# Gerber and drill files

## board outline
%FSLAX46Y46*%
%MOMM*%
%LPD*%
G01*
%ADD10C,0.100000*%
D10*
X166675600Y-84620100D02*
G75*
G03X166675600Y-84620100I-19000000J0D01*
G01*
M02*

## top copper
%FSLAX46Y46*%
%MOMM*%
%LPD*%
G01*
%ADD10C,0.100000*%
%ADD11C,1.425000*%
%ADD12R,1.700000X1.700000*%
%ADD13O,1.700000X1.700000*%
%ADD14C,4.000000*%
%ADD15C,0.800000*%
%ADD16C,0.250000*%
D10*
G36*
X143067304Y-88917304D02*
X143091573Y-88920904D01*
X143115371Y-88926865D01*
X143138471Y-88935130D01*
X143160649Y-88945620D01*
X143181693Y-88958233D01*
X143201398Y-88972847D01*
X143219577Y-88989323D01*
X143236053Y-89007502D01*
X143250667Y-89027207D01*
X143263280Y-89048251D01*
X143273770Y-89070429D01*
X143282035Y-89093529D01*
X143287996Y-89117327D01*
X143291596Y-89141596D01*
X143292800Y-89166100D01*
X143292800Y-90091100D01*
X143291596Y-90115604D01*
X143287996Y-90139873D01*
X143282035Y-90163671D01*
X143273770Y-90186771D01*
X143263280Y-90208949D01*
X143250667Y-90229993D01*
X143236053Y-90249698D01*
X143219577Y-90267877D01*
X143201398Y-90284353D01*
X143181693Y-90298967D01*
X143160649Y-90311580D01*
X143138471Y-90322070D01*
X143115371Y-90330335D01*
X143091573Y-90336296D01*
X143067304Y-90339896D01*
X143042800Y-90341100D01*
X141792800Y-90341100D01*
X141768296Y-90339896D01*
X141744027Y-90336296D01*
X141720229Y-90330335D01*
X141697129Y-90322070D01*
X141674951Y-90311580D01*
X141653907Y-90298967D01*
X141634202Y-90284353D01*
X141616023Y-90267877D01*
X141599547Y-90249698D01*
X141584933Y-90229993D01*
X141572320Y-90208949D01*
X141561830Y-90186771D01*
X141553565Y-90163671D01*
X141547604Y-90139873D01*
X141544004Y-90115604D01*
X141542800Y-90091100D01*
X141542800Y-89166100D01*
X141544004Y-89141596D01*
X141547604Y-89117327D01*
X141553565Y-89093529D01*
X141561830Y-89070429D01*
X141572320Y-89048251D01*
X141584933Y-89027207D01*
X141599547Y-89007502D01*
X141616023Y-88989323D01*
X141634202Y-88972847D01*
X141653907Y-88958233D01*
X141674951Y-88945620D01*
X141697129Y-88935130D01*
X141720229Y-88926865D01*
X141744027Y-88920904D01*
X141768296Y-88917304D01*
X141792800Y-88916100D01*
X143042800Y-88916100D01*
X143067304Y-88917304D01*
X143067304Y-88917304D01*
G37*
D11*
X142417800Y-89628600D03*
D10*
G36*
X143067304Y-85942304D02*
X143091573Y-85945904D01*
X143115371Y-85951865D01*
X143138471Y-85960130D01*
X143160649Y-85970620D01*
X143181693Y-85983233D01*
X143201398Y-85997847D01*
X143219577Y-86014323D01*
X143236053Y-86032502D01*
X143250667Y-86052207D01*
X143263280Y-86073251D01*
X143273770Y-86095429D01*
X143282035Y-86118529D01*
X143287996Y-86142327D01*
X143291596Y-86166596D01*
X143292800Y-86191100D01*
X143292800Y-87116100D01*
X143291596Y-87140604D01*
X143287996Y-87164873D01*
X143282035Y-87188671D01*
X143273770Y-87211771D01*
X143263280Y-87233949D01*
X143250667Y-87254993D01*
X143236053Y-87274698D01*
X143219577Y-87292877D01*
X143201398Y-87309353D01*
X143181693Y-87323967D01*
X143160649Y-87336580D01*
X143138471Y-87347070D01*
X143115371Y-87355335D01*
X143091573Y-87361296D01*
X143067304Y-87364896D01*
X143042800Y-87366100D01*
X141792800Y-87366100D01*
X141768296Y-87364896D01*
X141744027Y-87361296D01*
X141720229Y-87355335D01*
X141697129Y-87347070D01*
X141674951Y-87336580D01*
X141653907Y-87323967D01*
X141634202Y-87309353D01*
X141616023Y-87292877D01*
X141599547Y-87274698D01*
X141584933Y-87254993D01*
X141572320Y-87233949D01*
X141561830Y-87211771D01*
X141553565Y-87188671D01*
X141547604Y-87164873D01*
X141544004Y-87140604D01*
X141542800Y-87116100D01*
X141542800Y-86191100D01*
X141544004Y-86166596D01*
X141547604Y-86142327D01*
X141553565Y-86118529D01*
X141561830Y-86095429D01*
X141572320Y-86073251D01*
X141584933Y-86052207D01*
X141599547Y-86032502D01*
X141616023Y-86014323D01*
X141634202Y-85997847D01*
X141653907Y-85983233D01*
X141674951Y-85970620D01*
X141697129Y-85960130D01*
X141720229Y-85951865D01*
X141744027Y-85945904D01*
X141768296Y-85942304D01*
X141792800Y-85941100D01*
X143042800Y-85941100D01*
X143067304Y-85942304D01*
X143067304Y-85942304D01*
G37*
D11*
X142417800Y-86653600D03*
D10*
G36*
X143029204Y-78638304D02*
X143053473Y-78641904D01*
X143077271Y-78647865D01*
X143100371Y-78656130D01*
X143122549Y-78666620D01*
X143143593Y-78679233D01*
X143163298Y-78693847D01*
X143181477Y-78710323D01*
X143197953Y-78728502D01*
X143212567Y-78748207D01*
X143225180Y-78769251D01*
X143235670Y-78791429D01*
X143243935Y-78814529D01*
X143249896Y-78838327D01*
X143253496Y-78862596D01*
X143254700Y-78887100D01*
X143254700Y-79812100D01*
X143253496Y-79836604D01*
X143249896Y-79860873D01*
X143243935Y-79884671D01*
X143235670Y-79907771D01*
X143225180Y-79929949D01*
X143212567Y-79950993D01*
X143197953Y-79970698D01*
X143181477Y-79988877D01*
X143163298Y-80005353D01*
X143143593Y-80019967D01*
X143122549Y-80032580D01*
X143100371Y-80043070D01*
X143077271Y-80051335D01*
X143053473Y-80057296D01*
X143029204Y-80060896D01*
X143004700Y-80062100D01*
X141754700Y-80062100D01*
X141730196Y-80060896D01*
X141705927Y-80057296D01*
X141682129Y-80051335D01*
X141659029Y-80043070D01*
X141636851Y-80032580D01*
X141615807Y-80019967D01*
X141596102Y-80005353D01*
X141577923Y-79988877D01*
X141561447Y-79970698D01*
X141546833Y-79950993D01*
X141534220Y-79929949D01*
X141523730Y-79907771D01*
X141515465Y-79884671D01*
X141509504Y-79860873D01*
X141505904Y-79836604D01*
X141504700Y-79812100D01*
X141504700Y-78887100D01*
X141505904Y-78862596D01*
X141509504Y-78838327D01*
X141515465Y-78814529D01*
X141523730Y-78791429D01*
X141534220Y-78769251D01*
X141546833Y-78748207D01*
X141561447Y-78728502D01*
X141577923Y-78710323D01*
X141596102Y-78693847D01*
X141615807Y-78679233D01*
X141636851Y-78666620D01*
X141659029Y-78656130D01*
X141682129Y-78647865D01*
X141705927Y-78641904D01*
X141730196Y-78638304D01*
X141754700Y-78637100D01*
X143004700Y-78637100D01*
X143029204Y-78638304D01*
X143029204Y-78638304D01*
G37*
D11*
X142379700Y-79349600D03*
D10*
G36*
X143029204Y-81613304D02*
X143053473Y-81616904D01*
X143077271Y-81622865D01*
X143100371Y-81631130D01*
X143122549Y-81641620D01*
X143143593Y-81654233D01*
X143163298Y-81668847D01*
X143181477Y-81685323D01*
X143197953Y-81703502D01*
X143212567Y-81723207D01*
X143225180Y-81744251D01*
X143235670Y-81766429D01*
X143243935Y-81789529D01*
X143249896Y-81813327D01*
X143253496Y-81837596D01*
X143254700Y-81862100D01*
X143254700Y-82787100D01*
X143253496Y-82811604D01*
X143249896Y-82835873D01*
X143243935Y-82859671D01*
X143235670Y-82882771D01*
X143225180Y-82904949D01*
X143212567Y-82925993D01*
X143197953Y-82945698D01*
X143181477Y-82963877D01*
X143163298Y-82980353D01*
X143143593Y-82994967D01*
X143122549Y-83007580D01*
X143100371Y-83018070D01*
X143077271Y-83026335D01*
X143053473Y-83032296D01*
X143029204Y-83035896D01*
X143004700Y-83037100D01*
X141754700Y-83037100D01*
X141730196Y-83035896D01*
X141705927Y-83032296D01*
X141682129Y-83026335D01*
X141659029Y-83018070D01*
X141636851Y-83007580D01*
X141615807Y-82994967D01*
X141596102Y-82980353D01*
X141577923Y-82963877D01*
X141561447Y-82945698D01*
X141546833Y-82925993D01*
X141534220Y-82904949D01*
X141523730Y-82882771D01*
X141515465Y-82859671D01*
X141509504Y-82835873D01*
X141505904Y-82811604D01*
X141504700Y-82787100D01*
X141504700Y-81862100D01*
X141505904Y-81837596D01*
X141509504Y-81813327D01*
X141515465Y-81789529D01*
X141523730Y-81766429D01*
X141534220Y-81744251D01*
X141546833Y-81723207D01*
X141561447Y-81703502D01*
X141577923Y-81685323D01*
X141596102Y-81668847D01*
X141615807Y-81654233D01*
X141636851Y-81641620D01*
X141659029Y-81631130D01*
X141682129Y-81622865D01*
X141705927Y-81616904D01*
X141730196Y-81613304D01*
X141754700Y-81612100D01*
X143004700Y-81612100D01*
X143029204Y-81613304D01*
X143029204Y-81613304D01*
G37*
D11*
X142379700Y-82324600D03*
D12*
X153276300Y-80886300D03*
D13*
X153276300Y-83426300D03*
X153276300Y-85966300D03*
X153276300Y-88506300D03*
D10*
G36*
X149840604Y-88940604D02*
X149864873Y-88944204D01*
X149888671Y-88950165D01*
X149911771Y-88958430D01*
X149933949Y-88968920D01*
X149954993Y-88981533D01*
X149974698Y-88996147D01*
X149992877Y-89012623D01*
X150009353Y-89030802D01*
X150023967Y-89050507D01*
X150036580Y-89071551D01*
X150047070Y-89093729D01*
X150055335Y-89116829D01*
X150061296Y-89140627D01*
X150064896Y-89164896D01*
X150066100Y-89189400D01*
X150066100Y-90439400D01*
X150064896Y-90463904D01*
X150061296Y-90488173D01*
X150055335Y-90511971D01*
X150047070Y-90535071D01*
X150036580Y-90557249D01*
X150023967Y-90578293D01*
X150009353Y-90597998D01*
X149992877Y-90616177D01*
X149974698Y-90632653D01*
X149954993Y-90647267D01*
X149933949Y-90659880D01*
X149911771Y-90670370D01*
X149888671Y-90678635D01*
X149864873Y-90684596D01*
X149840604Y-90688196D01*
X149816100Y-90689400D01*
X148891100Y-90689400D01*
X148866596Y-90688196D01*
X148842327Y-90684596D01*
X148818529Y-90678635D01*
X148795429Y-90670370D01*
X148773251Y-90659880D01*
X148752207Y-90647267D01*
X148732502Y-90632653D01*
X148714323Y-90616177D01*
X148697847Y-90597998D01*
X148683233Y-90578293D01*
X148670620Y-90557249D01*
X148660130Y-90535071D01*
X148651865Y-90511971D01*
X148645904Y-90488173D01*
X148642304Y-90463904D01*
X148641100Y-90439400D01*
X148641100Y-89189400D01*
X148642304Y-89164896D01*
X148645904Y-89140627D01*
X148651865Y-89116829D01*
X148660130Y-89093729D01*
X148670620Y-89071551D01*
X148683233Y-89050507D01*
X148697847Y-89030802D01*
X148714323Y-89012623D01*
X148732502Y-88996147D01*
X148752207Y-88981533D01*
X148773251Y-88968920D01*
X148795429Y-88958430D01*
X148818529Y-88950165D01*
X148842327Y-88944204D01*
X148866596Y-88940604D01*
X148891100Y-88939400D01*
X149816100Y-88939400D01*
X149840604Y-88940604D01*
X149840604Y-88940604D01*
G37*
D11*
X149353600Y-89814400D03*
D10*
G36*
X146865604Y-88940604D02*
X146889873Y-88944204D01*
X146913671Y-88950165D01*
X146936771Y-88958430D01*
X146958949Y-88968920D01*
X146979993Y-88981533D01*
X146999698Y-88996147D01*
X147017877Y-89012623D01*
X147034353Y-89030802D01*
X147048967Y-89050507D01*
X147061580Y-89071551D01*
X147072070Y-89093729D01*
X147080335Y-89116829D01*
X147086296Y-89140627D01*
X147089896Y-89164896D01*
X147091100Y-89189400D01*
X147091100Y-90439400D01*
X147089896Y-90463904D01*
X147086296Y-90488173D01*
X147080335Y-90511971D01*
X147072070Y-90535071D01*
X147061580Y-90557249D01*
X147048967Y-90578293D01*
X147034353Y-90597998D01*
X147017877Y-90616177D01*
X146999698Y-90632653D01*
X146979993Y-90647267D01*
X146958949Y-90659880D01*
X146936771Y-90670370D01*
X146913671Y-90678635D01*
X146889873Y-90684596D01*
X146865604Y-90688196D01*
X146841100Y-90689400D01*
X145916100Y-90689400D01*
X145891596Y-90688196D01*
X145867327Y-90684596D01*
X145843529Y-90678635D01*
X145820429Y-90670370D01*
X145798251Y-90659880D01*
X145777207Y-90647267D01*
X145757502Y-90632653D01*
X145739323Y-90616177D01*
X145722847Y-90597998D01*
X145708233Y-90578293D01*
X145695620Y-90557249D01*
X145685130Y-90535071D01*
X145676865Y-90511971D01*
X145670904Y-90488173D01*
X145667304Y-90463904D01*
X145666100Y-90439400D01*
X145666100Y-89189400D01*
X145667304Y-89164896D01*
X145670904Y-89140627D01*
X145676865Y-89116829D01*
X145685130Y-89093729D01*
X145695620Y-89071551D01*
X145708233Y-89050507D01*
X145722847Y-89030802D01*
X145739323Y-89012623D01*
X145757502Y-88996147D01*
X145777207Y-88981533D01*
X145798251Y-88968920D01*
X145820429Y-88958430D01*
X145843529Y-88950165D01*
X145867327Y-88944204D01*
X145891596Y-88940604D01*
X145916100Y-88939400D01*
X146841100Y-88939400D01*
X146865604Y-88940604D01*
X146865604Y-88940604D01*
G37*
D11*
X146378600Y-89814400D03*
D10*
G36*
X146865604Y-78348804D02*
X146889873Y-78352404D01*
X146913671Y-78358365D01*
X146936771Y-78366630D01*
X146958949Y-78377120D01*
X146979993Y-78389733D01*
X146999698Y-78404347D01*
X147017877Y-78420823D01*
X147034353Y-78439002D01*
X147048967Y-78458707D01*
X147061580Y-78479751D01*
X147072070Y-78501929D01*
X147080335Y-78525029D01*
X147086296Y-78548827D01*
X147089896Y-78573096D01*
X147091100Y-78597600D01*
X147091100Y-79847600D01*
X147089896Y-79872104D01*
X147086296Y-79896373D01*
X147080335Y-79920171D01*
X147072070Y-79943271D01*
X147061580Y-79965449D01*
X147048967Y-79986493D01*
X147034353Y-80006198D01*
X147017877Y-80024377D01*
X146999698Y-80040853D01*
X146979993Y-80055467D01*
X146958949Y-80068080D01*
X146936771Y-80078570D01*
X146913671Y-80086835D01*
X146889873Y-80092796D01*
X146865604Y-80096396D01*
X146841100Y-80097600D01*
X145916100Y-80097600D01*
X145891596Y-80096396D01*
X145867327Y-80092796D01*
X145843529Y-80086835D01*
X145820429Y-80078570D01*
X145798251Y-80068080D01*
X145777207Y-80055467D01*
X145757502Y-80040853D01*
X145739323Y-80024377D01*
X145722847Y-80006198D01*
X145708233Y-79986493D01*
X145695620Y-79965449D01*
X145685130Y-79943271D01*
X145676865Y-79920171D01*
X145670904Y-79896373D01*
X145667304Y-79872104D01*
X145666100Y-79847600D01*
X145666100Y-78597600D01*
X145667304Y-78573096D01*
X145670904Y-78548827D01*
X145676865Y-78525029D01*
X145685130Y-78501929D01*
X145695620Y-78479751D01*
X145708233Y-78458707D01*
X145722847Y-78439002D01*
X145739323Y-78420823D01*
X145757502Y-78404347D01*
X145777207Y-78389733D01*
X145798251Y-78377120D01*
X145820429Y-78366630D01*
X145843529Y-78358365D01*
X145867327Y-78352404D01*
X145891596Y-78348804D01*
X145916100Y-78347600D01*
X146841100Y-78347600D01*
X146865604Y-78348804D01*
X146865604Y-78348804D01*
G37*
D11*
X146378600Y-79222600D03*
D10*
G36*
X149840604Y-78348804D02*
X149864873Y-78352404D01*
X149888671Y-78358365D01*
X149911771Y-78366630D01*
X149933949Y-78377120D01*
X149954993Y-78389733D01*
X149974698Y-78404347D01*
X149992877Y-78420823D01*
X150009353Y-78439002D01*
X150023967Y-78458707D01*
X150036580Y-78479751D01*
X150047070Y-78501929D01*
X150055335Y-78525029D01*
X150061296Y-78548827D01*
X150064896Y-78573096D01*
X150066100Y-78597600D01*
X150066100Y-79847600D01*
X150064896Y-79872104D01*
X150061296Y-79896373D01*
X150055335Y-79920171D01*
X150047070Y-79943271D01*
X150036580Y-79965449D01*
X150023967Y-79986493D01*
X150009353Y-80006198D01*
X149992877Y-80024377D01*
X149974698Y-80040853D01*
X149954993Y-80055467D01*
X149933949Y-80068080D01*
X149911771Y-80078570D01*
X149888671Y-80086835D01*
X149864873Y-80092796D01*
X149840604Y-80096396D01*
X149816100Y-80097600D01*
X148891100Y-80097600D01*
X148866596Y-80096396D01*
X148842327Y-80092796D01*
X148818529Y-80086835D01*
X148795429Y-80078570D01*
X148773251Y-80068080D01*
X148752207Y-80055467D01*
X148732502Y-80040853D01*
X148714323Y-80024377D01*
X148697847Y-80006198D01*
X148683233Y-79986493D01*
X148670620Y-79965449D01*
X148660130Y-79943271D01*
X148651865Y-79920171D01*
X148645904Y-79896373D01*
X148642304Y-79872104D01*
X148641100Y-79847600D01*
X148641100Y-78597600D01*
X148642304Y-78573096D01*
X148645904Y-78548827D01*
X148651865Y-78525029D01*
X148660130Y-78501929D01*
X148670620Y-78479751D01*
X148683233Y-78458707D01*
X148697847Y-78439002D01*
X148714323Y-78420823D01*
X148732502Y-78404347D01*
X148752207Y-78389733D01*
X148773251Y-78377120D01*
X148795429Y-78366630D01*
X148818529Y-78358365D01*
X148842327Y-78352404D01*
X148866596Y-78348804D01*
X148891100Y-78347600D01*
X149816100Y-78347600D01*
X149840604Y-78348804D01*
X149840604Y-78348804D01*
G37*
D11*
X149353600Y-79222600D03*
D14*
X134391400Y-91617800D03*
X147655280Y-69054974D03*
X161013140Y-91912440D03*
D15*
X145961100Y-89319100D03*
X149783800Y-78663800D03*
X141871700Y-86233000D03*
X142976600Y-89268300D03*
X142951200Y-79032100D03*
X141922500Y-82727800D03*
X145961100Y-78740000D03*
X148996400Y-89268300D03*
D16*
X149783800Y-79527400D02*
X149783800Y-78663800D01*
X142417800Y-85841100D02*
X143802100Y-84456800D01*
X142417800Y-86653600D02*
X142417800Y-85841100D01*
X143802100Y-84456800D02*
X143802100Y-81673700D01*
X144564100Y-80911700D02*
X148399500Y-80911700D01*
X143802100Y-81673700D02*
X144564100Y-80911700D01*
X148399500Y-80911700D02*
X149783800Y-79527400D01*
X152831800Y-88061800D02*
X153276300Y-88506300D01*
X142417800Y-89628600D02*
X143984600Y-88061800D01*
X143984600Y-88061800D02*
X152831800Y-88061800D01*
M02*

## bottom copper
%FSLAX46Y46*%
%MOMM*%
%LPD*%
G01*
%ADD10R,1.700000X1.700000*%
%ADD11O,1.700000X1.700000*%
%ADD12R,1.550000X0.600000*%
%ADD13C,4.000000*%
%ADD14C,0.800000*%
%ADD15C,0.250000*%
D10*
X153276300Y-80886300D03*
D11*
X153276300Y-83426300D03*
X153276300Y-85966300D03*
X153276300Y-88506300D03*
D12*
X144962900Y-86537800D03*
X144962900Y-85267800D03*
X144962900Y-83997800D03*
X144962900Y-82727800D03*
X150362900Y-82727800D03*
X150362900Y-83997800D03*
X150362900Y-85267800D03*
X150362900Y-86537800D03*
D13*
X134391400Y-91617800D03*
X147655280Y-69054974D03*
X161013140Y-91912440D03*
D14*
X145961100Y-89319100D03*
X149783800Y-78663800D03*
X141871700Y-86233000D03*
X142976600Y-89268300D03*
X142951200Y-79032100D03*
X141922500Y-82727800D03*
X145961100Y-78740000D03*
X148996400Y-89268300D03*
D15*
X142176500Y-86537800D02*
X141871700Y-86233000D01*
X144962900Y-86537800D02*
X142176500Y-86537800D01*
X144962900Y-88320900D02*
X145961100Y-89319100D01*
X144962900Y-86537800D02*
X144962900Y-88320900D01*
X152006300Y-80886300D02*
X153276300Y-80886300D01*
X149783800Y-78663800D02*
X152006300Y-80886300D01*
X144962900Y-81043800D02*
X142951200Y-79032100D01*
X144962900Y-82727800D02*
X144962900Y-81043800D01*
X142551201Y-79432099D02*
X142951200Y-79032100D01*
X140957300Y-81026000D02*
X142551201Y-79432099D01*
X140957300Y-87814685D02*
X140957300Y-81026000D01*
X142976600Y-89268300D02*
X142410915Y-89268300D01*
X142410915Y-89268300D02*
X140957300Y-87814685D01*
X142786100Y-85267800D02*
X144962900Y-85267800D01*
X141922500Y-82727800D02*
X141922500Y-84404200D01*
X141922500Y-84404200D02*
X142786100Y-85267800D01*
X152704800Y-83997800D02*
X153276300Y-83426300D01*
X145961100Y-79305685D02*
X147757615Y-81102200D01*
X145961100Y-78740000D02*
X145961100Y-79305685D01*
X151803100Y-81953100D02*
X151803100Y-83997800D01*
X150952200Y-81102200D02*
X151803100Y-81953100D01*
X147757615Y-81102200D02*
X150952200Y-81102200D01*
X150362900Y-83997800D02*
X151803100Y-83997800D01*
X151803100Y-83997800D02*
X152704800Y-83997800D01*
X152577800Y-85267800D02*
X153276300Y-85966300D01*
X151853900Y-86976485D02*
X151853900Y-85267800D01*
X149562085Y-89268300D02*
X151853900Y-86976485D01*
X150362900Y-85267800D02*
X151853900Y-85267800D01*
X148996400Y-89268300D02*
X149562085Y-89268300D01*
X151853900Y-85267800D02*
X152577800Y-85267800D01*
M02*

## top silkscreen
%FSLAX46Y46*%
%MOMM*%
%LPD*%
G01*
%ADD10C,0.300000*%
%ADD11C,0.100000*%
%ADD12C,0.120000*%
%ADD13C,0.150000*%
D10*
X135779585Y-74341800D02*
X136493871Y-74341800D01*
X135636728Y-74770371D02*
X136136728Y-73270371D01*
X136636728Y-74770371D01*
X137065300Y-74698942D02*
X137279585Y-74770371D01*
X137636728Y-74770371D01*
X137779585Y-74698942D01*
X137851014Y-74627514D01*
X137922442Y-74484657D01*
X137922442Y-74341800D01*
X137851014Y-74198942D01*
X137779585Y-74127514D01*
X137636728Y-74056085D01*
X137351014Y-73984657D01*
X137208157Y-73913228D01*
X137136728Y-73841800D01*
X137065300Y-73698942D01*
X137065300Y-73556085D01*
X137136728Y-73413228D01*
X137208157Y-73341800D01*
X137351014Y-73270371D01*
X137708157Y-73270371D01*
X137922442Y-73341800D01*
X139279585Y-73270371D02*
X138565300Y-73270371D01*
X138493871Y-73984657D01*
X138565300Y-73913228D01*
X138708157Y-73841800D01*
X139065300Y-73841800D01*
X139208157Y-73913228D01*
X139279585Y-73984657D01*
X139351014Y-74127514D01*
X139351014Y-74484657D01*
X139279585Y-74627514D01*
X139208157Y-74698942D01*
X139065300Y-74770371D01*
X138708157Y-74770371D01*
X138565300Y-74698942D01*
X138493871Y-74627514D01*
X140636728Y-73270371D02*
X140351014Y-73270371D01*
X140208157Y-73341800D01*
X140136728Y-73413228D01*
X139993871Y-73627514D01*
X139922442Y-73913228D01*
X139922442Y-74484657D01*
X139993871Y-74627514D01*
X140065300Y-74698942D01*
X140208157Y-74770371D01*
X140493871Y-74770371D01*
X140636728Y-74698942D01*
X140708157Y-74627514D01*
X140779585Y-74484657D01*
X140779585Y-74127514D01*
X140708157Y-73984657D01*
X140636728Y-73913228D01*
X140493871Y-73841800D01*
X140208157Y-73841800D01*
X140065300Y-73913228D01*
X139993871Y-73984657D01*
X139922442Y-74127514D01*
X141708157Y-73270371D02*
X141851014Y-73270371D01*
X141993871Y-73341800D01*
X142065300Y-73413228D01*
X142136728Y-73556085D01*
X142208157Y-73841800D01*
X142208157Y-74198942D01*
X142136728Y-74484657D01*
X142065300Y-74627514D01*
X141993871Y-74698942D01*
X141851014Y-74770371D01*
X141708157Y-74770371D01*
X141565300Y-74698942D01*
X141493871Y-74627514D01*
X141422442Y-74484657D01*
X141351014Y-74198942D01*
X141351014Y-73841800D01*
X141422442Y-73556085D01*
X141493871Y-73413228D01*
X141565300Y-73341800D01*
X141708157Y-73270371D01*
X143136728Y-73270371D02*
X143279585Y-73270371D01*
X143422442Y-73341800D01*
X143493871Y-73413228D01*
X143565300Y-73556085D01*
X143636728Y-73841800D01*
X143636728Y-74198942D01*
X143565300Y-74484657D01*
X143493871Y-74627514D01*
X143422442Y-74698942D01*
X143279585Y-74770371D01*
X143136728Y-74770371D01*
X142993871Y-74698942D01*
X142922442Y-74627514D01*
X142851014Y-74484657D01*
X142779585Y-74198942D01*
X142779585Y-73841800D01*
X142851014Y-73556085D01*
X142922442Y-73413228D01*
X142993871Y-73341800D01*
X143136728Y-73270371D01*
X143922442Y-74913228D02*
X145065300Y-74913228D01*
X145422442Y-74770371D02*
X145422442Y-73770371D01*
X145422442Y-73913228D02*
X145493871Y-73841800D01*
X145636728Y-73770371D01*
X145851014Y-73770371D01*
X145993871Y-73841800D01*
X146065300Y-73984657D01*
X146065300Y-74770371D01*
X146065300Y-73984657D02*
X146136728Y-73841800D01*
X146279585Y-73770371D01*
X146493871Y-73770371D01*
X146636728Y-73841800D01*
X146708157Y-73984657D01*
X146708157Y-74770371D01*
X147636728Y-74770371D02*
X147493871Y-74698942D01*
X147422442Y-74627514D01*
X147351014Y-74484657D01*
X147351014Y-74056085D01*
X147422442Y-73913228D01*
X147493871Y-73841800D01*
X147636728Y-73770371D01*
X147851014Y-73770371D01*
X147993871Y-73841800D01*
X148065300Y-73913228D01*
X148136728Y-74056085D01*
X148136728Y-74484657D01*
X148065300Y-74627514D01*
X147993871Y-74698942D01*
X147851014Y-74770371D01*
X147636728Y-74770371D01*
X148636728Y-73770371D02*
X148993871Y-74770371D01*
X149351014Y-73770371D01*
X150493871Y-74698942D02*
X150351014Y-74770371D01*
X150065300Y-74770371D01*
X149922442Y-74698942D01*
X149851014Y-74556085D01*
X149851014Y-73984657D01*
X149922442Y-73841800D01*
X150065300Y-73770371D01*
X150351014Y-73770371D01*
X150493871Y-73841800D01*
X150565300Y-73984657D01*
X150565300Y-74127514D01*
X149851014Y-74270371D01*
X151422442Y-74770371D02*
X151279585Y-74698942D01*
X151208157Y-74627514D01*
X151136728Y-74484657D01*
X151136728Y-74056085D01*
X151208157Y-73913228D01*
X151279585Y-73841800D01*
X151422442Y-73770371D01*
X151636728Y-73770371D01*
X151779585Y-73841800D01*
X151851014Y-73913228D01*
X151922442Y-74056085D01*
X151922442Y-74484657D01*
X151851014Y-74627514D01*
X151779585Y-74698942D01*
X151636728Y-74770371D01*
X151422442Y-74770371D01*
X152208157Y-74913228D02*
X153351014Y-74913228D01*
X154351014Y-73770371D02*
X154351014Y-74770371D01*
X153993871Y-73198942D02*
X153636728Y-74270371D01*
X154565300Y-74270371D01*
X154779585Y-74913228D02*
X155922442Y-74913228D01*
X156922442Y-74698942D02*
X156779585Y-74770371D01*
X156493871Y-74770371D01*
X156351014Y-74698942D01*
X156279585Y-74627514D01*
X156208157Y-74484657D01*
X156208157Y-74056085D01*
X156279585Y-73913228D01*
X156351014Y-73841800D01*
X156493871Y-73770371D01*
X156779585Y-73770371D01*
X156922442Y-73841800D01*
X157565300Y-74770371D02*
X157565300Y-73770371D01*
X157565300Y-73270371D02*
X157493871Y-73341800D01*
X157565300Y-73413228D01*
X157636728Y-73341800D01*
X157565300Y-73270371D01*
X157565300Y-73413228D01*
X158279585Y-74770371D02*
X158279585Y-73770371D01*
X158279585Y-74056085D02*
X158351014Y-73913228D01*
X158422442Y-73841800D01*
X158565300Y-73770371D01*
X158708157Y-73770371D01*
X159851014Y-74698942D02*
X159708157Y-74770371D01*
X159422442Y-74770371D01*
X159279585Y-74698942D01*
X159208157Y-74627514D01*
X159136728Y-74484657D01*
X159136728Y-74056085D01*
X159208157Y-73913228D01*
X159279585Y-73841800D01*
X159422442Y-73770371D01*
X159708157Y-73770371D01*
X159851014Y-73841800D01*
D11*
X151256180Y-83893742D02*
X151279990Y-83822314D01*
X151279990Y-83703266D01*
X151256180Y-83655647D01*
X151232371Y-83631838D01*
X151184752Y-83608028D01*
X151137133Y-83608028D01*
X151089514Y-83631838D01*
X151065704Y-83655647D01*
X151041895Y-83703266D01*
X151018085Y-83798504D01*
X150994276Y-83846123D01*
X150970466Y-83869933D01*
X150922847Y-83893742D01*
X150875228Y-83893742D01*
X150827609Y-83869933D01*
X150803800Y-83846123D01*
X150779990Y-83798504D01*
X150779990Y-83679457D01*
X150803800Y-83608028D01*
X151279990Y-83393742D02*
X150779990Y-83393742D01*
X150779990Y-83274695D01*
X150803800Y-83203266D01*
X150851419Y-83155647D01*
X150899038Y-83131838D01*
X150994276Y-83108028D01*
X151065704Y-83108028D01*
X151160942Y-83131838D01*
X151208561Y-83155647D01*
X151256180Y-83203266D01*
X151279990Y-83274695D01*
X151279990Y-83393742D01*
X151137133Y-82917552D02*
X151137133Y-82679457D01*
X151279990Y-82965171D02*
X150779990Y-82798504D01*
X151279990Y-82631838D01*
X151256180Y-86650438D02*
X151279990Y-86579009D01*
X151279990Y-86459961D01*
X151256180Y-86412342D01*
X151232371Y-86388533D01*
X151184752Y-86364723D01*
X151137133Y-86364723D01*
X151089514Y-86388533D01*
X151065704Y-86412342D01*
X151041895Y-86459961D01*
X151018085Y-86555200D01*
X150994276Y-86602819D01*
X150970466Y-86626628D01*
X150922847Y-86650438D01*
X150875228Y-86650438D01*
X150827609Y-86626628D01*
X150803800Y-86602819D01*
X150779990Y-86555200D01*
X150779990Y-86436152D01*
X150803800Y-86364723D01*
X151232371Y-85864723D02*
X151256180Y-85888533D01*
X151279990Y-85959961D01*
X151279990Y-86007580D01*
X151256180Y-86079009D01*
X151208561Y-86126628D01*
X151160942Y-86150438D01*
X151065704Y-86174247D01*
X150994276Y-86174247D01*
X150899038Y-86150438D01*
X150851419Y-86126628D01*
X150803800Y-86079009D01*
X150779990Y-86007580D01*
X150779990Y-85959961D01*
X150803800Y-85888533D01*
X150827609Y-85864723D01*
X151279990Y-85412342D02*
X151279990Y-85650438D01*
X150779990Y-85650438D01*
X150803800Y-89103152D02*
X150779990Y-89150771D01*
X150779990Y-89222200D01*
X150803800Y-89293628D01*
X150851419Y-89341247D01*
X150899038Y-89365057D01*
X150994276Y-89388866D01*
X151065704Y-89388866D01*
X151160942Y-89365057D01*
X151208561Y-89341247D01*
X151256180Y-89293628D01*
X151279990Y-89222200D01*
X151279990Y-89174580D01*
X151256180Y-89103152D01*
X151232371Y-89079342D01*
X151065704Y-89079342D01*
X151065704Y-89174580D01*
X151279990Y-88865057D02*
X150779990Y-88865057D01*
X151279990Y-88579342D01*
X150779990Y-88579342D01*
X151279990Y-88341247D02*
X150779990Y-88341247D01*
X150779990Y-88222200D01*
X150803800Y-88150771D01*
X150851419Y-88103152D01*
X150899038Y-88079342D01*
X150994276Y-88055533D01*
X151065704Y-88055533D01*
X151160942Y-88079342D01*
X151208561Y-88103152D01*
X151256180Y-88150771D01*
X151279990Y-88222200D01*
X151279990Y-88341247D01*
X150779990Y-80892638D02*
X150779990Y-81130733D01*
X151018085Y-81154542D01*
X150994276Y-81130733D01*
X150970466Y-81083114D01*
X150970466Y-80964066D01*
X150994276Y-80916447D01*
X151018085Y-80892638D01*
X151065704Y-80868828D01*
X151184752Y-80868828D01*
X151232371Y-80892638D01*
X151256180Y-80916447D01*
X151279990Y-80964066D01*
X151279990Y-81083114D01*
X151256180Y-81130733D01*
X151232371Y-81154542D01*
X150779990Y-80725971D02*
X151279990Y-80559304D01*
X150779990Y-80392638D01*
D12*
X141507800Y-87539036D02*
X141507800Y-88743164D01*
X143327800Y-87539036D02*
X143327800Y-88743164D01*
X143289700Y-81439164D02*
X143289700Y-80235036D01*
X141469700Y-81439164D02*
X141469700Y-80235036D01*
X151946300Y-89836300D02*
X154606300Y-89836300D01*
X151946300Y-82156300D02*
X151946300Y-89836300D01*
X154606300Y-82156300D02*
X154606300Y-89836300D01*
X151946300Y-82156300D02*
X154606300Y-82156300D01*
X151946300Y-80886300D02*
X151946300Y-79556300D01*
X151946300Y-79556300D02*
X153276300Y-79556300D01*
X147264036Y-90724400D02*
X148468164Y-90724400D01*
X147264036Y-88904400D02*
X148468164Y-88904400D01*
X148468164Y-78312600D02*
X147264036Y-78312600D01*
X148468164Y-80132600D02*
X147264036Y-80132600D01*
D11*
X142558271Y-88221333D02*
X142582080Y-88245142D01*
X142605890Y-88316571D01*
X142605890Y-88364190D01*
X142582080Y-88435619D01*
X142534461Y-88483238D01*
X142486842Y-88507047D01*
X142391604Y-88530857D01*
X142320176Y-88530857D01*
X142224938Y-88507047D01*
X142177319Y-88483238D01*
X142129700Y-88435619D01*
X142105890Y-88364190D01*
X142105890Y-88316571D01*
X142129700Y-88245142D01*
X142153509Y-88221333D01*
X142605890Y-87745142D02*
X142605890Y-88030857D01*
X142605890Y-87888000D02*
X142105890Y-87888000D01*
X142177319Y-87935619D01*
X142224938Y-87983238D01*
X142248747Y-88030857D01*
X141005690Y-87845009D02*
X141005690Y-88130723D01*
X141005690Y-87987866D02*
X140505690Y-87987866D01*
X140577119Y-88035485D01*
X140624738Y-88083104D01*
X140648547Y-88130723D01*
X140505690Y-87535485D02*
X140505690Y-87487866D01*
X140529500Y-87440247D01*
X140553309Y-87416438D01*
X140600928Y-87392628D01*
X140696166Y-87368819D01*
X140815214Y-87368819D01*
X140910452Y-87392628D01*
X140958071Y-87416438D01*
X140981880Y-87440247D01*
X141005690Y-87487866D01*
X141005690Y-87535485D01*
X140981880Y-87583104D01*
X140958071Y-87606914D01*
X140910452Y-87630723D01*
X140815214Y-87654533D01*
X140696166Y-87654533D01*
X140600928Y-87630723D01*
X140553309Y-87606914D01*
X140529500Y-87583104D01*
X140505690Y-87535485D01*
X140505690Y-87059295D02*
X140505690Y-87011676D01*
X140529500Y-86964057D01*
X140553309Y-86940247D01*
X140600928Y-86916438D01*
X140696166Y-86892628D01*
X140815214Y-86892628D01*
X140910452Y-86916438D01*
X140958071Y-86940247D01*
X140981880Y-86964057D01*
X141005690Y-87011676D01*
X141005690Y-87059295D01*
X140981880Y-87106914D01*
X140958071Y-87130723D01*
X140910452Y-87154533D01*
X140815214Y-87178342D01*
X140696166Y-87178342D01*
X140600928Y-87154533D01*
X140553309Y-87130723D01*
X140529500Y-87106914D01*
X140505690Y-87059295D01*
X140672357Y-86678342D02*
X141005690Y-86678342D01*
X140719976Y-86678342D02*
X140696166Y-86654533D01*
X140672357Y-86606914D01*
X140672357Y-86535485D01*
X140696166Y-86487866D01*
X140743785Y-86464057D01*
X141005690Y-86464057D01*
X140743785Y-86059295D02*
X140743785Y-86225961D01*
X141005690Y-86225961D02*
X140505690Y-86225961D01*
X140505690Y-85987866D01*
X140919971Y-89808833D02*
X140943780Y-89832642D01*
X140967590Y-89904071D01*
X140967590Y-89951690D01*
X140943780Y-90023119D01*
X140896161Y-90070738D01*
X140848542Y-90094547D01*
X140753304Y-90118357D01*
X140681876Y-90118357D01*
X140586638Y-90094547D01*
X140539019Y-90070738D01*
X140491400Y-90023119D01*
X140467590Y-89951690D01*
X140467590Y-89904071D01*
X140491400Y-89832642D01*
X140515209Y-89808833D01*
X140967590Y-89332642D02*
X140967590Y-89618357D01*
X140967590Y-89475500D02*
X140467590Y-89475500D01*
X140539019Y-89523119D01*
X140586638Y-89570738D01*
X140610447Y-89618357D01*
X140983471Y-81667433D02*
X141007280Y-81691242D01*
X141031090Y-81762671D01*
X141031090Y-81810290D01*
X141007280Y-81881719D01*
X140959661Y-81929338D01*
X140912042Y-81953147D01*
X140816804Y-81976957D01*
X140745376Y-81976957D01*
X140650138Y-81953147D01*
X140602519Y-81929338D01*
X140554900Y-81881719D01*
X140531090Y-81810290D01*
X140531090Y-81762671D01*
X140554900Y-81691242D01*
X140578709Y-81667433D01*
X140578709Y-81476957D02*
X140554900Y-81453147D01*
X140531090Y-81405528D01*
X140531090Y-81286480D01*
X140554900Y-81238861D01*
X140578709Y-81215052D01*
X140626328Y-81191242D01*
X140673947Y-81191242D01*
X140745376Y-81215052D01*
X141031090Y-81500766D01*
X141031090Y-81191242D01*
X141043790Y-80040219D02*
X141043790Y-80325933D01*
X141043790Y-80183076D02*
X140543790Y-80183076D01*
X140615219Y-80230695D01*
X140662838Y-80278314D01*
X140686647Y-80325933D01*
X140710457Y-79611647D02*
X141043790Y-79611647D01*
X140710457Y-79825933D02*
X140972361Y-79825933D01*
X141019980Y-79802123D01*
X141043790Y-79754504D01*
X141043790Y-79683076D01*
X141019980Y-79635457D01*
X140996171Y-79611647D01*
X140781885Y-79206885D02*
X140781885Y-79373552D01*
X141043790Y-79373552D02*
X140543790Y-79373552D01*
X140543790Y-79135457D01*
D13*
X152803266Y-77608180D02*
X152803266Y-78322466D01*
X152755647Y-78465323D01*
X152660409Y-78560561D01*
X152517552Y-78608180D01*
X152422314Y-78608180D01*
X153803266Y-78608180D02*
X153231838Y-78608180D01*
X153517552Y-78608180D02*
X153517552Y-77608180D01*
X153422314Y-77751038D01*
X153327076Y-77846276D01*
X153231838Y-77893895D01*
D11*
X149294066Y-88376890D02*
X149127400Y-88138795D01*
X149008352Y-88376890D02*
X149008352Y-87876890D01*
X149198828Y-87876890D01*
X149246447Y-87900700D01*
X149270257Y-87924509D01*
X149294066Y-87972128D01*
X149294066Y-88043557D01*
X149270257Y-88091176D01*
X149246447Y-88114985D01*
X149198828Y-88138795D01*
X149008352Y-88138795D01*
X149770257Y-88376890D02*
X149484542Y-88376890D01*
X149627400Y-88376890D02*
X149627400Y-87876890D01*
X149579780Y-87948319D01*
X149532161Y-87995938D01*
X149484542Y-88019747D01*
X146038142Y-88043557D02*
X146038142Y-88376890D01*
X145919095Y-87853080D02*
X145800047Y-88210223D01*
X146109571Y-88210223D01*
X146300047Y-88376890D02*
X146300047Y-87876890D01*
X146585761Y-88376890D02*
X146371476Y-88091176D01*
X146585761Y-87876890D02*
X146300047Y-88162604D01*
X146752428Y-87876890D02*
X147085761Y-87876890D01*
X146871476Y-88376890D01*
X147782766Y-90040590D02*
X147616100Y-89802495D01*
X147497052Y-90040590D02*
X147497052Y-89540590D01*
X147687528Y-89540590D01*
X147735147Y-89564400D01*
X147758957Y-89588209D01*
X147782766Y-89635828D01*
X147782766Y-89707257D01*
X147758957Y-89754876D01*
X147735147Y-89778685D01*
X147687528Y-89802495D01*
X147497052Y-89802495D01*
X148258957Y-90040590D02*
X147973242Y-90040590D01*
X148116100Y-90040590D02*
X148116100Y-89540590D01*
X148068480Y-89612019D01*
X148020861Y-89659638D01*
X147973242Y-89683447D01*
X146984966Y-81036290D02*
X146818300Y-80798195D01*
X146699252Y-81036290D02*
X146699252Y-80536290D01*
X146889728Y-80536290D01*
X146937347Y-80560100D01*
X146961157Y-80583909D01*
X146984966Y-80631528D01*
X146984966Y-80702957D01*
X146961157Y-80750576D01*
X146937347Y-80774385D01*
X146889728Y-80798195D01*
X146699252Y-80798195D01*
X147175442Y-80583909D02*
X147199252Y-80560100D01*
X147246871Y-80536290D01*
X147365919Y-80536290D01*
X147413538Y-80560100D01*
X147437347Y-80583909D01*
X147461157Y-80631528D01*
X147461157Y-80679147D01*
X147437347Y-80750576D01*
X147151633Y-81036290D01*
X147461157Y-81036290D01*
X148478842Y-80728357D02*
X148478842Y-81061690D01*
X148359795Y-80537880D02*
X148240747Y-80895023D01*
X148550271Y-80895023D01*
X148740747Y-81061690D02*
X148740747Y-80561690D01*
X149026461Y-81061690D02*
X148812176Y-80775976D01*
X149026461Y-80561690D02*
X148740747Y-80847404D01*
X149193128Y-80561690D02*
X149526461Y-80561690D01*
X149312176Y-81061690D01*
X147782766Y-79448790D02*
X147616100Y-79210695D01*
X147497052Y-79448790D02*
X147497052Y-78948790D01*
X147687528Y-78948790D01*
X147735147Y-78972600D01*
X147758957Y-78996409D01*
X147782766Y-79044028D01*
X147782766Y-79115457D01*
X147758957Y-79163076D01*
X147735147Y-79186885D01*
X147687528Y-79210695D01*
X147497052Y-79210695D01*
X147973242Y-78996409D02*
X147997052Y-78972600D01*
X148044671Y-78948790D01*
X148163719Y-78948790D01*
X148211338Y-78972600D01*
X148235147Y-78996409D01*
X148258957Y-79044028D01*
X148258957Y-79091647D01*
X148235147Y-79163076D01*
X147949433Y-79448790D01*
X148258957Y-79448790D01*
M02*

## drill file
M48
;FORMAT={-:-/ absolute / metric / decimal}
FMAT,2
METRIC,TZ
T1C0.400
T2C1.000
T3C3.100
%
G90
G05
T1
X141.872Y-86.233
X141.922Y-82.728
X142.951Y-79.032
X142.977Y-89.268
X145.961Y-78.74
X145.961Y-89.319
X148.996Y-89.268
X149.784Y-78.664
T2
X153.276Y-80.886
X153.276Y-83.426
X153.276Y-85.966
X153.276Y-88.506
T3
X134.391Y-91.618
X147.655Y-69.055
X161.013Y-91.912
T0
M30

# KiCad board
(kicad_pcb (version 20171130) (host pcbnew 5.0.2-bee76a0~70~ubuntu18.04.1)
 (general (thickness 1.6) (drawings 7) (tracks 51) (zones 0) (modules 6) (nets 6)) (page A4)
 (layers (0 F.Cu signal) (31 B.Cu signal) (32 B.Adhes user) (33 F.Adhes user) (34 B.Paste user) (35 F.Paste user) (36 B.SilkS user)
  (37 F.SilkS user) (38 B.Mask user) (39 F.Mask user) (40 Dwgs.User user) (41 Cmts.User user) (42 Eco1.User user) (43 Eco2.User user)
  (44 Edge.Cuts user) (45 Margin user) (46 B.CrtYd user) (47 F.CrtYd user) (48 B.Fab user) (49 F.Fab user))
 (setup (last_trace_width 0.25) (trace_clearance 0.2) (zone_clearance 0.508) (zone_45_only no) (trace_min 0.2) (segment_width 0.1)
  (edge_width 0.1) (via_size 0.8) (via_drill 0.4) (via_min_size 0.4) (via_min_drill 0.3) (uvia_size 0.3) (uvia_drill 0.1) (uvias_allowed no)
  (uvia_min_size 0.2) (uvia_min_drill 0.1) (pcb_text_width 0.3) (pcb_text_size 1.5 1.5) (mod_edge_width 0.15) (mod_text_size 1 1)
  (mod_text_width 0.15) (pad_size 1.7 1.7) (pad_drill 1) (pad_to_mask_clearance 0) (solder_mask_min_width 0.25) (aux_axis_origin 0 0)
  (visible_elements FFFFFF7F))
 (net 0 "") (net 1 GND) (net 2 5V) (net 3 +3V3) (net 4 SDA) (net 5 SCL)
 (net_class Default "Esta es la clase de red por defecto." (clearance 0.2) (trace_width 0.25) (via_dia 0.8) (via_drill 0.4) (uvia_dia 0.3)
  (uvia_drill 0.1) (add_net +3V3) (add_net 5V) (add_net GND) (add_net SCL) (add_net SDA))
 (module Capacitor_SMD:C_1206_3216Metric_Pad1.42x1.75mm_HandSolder (layer F.Cu) (at 142.4178 88.1411 270)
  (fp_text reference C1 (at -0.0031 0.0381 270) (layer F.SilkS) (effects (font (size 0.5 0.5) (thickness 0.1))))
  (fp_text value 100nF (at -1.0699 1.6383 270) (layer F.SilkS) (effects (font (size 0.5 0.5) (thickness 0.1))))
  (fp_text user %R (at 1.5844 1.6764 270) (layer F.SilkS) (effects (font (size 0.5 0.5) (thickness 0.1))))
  (fp_line (start -0.602064 0.91) (end 0.602064 0.91) (layer F.SilkS) (width 0.12))
  (fp_line (start -0.602064 -0.91) (end 0.602064 -0.91) (layer F.SilkS) (width 0.12))
  (pad 2 smd roundrect (at 1.4875 0 270) (size 1.425 1.75) (layers F.Cu F.Paste F.Mask) (roundrect_rratio 0.175439) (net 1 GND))
  (pad 1 smd roundrect (at -1.4875 0 270) (size 1.425 1.75) (layers F.Cu F.Paste F.Mask) (roundrect_rratio 0.175439) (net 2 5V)))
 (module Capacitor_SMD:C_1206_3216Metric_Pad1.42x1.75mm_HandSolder (layer F.Cu) (at 142.3797 80.8371 90)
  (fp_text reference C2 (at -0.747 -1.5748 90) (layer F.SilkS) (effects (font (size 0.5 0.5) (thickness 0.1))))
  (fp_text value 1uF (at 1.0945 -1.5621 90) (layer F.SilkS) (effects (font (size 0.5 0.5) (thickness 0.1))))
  (fp_line (start -0.602064 0.91) (end 0.602064 0.91) (layer F.SilkS) (width 0.12))
  (fp_line (start -0.602064 -0.91) (end 0.602064 -0.91) (layer F.SilkS) (width 0.12))
  (pad 2 smd roundrect (at 1.4875 0 90) (size 1.425 1.75) (layers F.Cu F.Paste F.Mask) (roundrect_rratio 0.175439) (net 1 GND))
  (pad 1 smd roundrect (at -1.4875 0 90) (size 1.425 1.75) (layers F.Cu F.Paste F.Mask) (roundrect_rratio 0.175439) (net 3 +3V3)))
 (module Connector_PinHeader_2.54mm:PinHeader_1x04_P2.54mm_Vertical (layer F.Cu) (at 153.2763 80.8863)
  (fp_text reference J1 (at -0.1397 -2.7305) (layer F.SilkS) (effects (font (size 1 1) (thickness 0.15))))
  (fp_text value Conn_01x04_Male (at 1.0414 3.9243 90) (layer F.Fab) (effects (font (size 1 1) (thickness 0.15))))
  (fp_line (start -1.33 8.95) (end 1.33 8.95) (layer F.SilkS) (width 0.12))
  (fp_line (start -1.33 1.27) (end -1.33 8.95) (layer F.SilkS) (width 0.12))
  (fp_line (start 1.33 1.27) (end 1.33 8.95) (layer F.SilkS) (width 0.12))
  (fp_line (start -1.33 1.27) (end 1.33 1.27) (layer F.SilkS) (width 0.12))
  (fp_line (start -1.33 0) (end -1.33 -1.33) (layer F.SilkS) (width 0.12))
  (fp_line (start -1.33 -1.33) (end 0 -1.33) (layer F.SilkS) (width 0.12))
  (pad 1 thru_hole rect (at 0 0) (size 1.7 1.7) (drill 1) (layers *.Cu *.Mask) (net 2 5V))
  (pad 2 thru_hole oval (at 0 2.54) (size 1.7 1.7) (drill 1) (layers *.Cu *.Mask) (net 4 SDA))
  (pad 3 thru_hole oval (at 0 5.08) (size 1.7 1.7) (drill 1) (layers *.Cu *.Mask) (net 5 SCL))
  (pad 4 thru_hole oval (at 0 7.62) (size 1.7 1.7) (drill 1) (layers *.Cu *.Mask) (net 1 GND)))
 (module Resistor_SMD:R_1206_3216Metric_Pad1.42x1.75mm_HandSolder (layer F.Cu) (at 147.8661 89.8144)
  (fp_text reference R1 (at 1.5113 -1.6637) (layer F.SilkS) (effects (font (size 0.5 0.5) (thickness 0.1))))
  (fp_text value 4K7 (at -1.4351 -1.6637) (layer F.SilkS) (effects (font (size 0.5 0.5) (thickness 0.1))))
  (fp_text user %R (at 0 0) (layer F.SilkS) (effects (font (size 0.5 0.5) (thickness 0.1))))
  (fp_line (start -0.602064 0.91) (end 0.602064 0.91) (layer F.SilkS) (width 0.12))
  (fp_line (start -0.602064 -0.91) (end 0.602064 -0.91) (layer F.SilkS) (width 0.12))
  (pad 2 smd roundrect (at 1.4875 0) (size 1.425 1.75) (layers F.Cu F.Paste F.Mask) (roundrect_rratio 0.175439) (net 5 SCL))
  (pad 1 smd roundrect (at -1.4875 0) (size 1.425 1.75) (layers F.Cu F.Paste F.Mask) (roundrect_rratio 0.175439) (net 2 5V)))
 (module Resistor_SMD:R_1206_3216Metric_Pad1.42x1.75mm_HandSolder (layer F.Cu) (at 147.8661 79.2226 180)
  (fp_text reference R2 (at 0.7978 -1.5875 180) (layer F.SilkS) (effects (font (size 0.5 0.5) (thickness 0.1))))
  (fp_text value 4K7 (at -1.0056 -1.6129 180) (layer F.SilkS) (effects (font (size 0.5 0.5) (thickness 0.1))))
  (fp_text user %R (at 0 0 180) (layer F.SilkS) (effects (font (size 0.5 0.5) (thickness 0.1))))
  (fp_line (start -0.602064 0.91) (end 0.602064 0.91) (layer F.SilkS) (width 0.12))
  (fp_line (start -0.602064 -0.91) (end 0.602064 -0.91) (layer F.SilkS) (width 0.12))
  (pad 2 smd roundrect (at 1.4875 0 180) (size 1.425 1.75) (layers F.Cu F.Paste F.Mask) (roundrect_rratio 0.175439) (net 4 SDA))
  (pad 1 smd roundrect (at -1.4875 0 180) (size 1.425 1.75) (layers F.Cu F.Paste F.Mask) (roundrect_rratio 0.175439) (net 2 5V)))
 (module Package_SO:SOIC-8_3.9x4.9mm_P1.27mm (layer B.Cu) (at 147.6629 84.6328)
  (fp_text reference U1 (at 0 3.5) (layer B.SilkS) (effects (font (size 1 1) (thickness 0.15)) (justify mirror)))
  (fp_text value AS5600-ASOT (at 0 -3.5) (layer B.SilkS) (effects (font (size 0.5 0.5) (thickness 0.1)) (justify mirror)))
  (pad 1 smd rect (at -2.7 1.905) (size 1.55 0.6) (layers B.Cu B.Paste B.Mask) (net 2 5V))
  (pad 2 smd rect (at -2.7 0.635) (size 1.55 0.6) (layers B.Cu B.Paste B.Mask) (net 3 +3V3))
  (pad 3 smd rect (at -2.7 -0.635) (size 1.55 0.6) (layers B.Cu B.Paste B.Mask))
  (pad 4 smd rect (at -2.7 -1.905) (size 1.55 0.6) (layers B.Cu B.Paste B.Mask) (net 1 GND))
  (pad 5 smd rect (at 2.7 -1.905) (size 1.55 0.6) (layers B.Cu B.Paste B.Mask))
  (pad 6 smd rect (at 2.7 -0.635) (size 1.55 0.6) (layers B.Cu B.Paste B.Mask) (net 4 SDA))
  (pad 7 smd rect (at 2.7 0.635) (size 1.55 0.6) (layers B.Cu B.Paste B.Mask) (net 5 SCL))
  (pad 8 smd rect (at 2.7 1.905) (size 1.55 0.6) (layers B.Cu B.Paste B.Mask)))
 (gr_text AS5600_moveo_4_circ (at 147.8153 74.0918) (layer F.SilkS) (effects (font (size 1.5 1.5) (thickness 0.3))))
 (gr_circle (center 147.6756 84.6201) (end 166.6756 84.6201) (layer Edge.Cuts) (width 0.1))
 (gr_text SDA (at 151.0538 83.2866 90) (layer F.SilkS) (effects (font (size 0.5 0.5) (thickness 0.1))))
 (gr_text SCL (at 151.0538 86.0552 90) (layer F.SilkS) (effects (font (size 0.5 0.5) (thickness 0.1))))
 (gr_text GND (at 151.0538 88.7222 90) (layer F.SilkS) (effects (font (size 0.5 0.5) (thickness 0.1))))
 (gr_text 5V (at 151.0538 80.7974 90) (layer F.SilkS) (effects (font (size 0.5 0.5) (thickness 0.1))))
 (via (at 134.3914 91.6178) (size 4) (drill 3.1) (layers F.Cu B.Cu) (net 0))
 (via (at 147.65528 69.054974) (size 4) (drill 3.1) (layers F.Cu B.Cu) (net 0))
 (via (at 161.01314 91.91244) (size 4) (drill 3.1) (layers F.Cu B.Cu) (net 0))
 (via (at 145.9611 89.3191) (size 0.8) (drill 0.4) (layers F.Cu B.Cu) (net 2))
 (via (at 149.7838 78.6638) (size 0.8) (drill 0.4) (layers F.Cu B.Cu) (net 2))
 (via (at 141.8717 86.233) (size 0.8) (drill 0.4) (layers F.Cu B.Cu) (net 2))
 (segment (start 142.1765 86.5378) (end 141.8717 86.233) (width 0.25) (layer B.Cu) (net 2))
 (segment (start 144.9629 86.5378) (end 142.1765 86.5378) (width 0.25) (layer B.Cu) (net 2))
 (segment (start 144.9629 88.3209) (end 145.9611 89.3191) (width 0.25) (layer B.Cu) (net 2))
 (segment (start 144.9629 86.5378) (end 144.9629 88.3209) (width 0.25) (layer B.Cu) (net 2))
 (segment (start 152.0063 80.8863) (end 153.2763 80.8863) (width 0.25) (layer B.Cu) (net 2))
 (segment (start 149.7838 78.6638) (end 152.0063 80.8863) (width 0.25) (layer B.Cu) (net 2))
 (segment (start 149.7838 79.5274) (end 149.7838 78.6638) (width 0.25) (layer F.Cu) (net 2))
 (segment (start 142.4178 85.8411) (end 143.8021 84.4568) (width 0.25) (layer F.Cu) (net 2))
 (segment (start 142.4178 86.6536) (end 142.4178 85.8411) (width 0.25) (layer F.Cu) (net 2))
 (segment (start 143.8021 84.4568) (end 143.8021 81.6737) (width 0.25) (layer F.Cu) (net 2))
 (segment (start 144.5641 80.9117) (end 148.3995 80.9117) (width 0.25) (layer F.Cu) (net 2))
 (segment (start 143.8021 81.6737) (end 144.5641 80.9117) (width 0.25) (layer F.Cu) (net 2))
 (segment (start 148.3995 80.9117) (end 149.7838 79.5274) (width 0.25) (layer F.Cu) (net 2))
 (via (at 142.9766 89.2683) (size 0.8) (drill 0.4) (layers F.Cu B.Cu) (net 1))
 (via (at 142.9512 79.0321) (size 0.8) (drill 0.4) (layers F.Cu B.Cu) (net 1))
 (segment (start 144.9629 81.0438) (end 142.9512 79.0321) (width 0.25) (layer B.Cu) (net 1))
 (segment (start 144.9629 82.7278) (end 144.9629 81.0438) (width 0.25) (layer B.Cu) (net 1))
 (segment (start 152.8318 88.0618) (end 153.2763 88.5063) (width 0.25) (layer F.Cu) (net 1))
 (segment (start 142.4178 89.6286) (end 143.9846 88.0618) (width 0.25) (layer F.Cu) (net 1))
 (segment (start 143.9846 88.0618) (end 152.8318 88.0618) (width 0.25) (layer F.Cu) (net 1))
 (segment (start 142.551201 79.432099) (end 142.9512 79.0321) (width 0.25) (layer B.Cu) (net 1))
 (segment (start 140.9573 81.026) (end 142.551201 79.432099) (width 0.25) (layer B.Cu) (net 1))
 (segment (start 140.9573 87.814685) (end 140.9573 81.026) (width 0.25) (layer B.Cu) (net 1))
 (segment (start 142.9766 89.2683) (end 142.410915 89.2683) (width 0.25) (layer B.Cu) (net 1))
 (segment (start 142.410915 89.2683) (end 140.9573 87.814685) (width 0.25) (layer B.Cu) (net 1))
 (via (at 141.9225 82.7278) (size 0.8) (drill 0.4) (layers F.Cu B.Cu) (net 3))
 (segment (start 142.7861 85.2678) (end 144.9629 85.2678) (width 0.25) (layer B.Cu) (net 3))
 (segment (start 141.9225 82.7278) (end 141.9225 84.4042) (width 0.25) (layer B.Cu) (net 3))
 (segment (start 141.9225 84.4042) (end 142.7861 85.2678) (width 0.25) (layer B.Cu) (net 3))
 (via (at 145.9611 78.74) (size 0.8) (drill 0.4) (layers F.Cu B.Cu) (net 4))
 (segment (start 152.7048 83.9978) (end 153.2763 83.4263) (width 0.25) (layer B.Cu) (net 4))
 (segment (start 145.9611 79.305685) (end 147.757615 81.1022) (width 0.25) (layer B.Cu) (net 4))
 (segment (start 145.9611 78.74) (end 145.9611 79.305685) (width 0.25) (layer B.Cu) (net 4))
 (segment (start 151.8031 81.9531) (end 151.8031 83.9978) (width 0.25) (layer B.Cu) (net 4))
 (segment (start 150.9522 81.1022) (end 151.8031 81.9531) (width 0.25) (layer B.Cu) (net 4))
 (segment (start 147.757615 81.1022) (end 150.9522 81.1022) (width 0.25) (layer B.Cu) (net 4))
 (segment (start 150.3629 83.9978) (end 151.8031 83.9978) (width 0.25) (layer B.Cu) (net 4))
 (segment (start 151.8031 83.9978) (end 152.7048 83.9978) (width 0.25) (layer B.Cu) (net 4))
 (via (at 148.9964 89.2683) (size 0.8) (drill 0.4) (layers F.Cu B.Cu) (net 5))
 (segment (start 152.5778 85.2678) (end 153.2763 85.9663) (width 0.25) (layer B.Cu) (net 5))
 (segment (start 151.8539 86.976485) (end 151.8539 85.2678) (width 0.25) (layer B.Cu) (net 5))
 (segment (start 149.562085 89.2683) (end 151.8539 86.976485) (width 0.25) (layer B.Cu) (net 5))
 (segment (start 150.3629 85.2678) (end 151.8539 85.2678) (width 0.25) (layer B.Cu) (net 5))
 (segment (start 148.9964 89.2683) (end 149.562085 89.2683) (width 0.25) (layer B.Cu) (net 5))
 (segment (start 151.8539 85.2678) (end 152.5778 85.2678) (width 0.25) (layer B.Cu) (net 5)))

